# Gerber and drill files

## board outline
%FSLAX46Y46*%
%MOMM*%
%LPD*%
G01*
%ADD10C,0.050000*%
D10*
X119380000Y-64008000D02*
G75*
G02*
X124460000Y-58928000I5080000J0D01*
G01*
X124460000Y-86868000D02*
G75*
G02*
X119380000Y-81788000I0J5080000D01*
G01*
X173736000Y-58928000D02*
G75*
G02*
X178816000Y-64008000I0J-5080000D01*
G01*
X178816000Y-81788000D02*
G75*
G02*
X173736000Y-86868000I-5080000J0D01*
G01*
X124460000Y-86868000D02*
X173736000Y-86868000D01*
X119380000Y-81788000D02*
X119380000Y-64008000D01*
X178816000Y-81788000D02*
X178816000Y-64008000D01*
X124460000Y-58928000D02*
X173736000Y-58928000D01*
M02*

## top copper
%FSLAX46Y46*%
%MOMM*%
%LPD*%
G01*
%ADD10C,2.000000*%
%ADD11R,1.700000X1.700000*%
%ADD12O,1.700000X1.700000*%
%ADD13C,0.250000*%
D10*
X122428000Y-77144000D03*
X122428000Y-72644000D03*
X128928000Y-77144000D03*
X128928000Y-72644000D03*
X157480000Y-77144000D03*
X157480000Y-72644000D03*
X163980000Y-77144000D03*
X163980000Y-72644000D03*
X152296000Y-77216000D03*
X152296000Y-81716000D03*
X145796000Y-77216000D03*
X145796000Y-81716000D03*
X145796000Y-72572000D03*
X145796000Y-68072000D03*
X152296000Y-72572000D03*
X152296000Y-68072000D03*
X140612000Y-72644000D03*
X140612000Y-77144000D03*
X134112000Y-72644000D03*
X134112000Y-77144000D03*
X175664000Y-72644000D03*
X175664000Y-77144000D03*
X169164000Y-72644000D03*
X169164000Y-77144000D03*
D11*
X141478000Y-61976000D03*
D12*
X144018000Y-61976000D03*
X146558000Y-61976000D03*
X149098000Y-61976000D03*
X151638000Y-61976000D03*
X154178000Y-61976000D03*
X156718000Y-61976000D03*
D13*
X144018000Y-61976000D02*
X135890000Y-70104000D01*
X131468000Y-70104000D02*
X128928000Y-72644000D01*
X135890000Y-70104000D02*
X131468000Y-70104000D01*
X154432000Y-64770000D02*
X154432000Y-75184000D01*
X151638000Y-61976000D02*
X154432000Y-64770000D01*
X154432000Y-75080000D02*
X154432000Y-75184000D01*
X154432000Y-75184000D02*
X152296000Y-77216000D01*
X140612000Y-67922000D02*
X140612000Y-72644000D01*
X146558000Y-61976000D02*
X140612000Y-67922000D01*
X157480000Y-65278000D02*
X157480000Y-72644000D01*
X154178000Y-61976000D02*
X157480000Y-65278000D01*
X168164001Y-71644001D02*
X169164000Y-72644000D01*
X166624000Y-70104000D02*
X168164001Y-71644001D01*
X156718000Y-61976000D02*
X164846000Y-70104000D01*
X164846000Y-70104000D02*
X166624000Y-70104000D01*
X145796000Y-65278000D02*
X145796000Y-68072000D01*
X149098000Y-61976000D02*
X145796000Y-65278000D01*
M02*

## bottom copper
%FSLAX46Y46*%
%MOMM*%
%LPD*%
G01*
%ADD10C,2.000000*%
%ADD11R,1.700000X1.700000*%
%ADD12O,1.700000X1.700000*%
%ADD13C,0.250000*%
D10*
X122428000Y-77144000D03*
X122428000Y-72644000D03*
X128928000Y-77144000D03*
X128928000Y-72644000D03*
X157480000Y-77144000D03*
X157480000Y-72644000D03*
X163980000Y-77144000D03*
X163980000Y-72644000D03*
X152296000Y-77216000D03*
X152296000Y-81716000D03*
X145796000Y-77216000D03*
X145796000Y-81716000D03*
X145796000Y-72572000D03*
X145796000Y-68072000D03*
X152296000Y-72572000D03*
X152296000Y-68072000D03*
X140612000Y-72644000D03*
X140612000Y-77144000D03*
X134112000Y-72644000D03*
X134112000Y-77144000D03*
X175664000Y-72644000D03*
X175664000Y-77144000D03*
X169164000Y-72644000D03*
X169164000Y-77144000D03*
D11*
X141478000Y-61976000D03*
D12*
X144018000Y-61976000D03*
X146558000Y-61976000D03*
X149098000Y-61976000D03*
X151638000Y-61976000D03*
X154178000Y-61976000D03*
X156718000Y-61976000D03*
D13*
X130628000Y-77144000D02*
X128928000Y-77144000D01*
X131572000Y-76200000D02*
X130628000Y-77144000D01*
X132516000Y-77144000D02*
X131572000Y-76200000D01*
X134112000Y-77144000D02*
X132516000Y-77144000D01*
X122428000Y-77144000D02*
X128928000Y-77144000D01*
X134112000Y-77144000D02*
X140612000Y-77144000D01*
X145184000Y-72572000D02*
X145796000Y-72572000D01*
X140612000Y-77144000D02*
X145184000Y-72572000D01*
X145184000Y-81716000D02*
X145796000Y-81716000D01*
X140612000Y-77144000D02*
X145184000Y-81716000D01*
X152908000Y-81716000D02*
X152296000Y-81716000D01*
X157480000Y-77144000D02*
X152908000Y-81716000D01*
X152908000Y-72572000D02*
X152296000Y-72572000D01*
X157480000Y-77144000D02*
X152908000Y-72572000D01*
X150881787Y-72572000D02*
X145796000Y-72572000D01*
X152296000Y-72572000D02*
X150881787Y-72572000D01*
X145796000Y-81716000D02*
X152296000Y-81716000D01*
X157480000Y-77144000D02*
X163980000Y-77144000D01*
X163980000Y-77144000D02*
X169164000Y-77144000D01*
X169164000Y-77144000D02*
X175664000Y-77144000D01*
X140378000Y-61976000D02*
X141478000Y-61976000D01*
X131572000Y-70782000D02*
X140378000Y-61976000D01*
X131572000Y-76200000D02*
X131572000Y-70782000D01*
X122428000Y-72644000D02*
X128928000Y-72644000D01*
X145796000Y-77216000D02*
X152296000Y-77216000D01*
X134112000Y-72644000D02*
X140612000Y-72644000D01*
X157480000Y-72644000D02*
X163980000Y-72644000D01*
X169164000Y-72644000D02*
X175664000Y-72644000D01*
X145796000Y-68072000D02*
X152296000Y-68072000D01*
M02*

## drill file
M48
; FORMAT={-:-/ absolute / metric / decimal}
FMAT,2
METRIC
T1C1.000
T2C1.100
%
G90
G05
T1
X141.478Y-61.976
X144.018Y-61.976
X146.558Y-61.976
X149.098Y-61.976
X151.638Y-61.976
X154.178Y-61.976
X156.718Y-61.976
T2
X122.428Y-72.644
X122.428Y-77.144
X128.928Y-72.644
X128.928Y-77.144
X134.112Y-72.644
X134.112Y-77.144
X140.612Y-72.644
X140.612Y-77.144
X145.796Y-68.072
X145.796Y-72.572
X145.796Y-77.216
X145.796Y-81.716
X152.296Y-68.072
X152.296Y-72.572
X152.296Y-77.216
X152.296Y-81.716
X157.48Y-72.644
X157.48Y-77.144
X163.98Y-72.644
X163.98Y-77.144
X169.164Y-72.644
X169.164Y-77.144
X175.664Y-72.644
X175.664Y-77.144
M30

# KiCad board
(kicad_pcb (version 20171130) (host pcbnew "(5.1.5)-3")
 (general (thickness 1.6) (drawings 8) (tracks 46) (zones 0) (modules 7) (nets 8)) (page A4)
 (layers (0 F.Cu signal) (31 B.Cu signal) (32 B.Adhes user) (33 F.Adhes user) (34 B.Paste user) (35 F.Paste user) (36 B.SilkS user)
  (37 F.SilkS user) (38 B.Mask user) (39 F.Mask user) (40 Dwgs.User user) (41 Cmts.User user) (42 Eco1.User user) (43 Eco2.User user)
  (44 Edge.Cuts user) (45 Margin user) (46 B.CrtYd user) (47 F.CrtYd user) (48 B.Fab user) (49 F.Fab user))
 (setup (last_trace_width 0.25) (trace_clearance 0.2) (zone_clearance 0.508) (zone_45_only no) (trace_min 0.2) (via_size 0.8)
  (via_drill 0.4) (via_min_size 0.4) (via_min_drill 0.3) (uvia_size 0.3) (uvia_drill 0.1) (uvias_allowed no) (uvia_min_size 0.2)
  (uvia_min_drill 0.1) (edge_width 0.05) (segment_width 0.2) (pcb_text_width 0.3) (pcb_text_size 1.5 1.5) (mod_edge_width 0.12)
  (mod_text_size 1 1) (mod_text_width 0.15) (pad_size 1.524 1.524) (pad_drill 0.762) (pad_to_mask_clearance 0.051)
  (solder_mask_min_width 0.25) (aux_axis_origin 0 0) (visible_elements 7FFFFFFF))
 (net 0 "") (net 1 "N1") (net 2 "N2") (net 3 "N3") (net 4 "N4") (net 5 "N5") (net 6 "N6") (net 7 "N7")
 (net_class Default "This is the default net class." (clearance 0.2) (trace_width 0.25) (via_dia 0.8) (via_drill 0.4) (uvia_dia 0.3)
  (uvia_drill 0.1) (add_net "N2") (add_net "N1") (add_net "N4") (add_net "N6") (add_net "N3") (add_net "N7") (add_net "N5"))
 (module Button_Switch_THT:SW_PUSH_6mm (layer F.Cu) (at 122.428 72.644)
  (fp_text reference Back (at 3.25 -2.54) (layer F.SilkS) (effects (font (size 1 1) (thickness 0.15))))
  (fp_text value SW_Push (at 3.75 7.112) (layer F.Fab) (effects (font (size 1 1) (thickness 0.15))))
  (pad 2 thru_hole circle (at 0 4.5 90) (size 2 2) (drill 1.1) (layers *.Cu *.Mask) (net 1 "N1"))
  (pad 1 thru_hole circle (at 0 0 90) (size 2 2) (drill 1.1) (layers *.Cu *.Mask) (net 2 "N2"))
  (pad 2 thru_hole circle (at 6.5 4.5 90) (size 2 2) (drill 1.1) (layers *.Cu *.Mask) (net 1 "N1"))
  (pad 1 thru_hole circle (at 6.5 0 90) (size 2 2) (drill 1.1) (layers *.Cu *.Mask) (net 2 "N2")))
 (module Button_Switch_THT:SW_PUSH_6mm (layer F.Cu) (at 157.48 72.644)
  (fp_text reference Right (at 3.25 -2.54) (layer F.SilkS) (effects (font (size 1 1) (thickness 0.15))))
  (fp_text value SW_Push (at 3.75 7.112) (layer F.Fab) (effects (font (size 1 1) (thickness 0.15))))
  (pad 2 thru_hole circle (at 0 4.5 90) (size 2 2) (drill 1.1) (layers *.Cu *.Mask) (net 1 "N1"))
  (pad 1 thru_hole circle (at 0 0 90) (size 2 2) (drill 1.1) (layers *.Cu *.Mask) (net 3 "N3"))
  (pad 2 thru_hole circle (at 6.5 4.5 90) (size 2 2) (drill 1.1) (layers *.Cu *.Mask) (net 1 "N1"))
  (pad 1 thru_hole circle (at 6.5 0 90) (size 2 2) (drill 1.1) (layers *.Cu *.Mask) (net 3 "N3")))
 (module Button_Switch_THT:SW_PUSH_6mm (layer F.Cu) (at 145.796 77.216)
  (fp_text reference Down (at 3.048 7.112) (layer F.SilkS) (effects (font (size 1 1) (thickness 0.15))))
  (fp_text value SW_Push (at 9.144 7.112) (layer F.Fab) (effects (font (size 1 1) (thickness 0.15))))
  (pad 1 thru_hole circle (at 6.5 0 90) (size 2 2) (drill 1.1) (layers *.Cu *.Mask) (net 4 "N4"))
  (pad 2 thru_hole circle (at 6.5 4.5 90) (size 2 2) (drill 1.1) (layers *.Cu *.Mask) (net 1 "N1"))
  (pad 1 thru_hole circle (at 0 0 90) (size 2 2) (drill 1.1) (layers *.Cu *.Mask) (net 4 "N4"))
  (pad 2 thru_hole circle (at 0 4.5 90) (size 2 2) (drill 1.1) (layers *.Cu *.Mask) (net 1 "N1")))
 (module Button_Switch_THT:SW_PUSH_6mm (layer F.Cu) (at 145.796 68.072)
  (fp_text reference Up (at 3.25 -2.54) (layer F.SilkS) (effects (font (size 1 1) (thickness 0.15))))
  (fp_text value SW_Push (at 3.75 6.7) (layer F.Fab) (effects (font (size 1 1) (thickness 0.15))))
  (pad 2 thru_hole circle (at 0 4.5 90) (size 2 2) (drill 1.1) (layers *.Cu *.Mask) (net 1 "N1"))
  (pad 1 thru_hole circle (at 0 0 90) (size 2 2) (drill 1.1) (layers *.Cu *.Mask) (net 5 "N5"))
  (pad 2 thru_hole circle (at 6.5 4.5 90) (size 2 2) (drill 1.1) (layers *.Cu *.Mask) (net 1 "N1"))
  (pad 1 thru_hole circle (at 6.5 0 90) (size 2 2) (drill 1.1) (layers *.Cu *.Mask) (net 5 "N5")))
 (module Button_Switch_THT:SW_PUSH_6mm (layer F.Cu) (at 134.112 72.644)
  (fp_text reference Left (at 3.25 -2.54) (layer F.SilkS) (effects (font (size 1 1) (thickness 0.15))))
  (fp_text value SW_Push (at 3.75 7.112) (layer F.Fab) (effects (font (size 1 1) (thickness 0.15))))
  (pad 1 thru_hole circle (at 6.5 0 90) (size 2 2) (drill 1.1) (layers *.Cu *.Mask) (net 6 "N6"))
  (pad 2 thru_hole circle (at 6.5 4.5 90) (size 2 2) (drill 1.1) (layers *.Cu *.Mask) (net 1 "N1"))
  (pad 1 thru_hole circle (at 0 0 90) (size 2 2) (drill 1.1) (layers *.Cu *.Mask) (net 6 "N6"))
  (pad 2 thru_hole circle (at 0 4.5 90) (size 2 2) (drill 1.1) (layers *.Cu *.Mask) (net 1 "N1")))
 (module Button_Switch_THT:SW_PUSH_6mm (layer F.Cu) (at 169.164 72.644)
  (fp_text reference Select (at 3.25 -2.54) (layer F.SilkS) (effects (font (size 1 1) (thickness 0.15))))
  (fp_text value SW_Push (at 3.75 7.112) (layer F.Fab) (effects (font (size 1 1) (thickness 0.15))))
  (pad 1 thru_hole circle (at 6.5 0 90) (size 2 2) (drill 1.1) (layers *.Cu *.Mask) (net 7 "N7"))
  (pad 2 thru_hole circle (at 6.5 4.5 90) (size 2 2) (drill 1.1) (layers *.Cu *.Mask) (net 1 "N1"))
  (pad 1 thru_hole circle (at 0 0 90) (size 2 2) (drill 1.1) (layers *.Cu *.Mask) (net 7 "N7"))
  (pad 2 thru_hole circle (at 0 4.5 90) (size 2 2) (drill 1.1) (layers *.Cu *.Mask) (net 1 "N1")))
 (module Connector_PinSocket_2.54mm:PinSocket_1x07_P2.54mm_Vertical (layer F.Cu) (at 141.478 61.976 90)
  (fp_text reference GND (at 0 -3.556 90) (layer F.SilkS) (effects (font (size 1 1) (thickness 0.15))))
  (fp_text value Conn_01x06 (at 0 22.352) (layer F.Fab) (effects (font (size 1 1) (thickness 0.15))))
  (pad 1 thru_hole rect (at 0 0 90) (size 1.7 1.7) (drill 1) (layers *.Cu *.Mask) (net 1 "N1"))
  (pad 2 thru_hole oval (at 0 2.54 90) (size 1.7 1.7) (drill 1) (layers *.Cu *.Mask) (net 2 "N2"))
  (pad 3 thru_hole oval (at 0 5.08 90) (size 1.7 1.7) (drill 1) (layers *.Cu *.Mask) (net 6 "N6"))
  (pad 4 thru_hole oval (at 0 7.62 90) (size 1.7 1.7) (drill 1) (layers *.Cu *.Mask) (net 5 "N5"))
  (pad 5 thru_hole oval (at 0 10.16 90) (size 1.7 1.7) (drill 1) (layers *.Cu *.Mask) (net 4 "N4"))
  (pad 6 thru_hole oval (at 0 12.7 90) (size 1.7 1.7) (drill 1) (layers *.Cu *.Mask) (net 3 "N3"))
  (pad 7 thru_hole oval (at 0 15.24 90) (size 1.7 1.7) (drill 1) (layers *.Cu *.Mask) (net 7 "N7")))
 (gr_arc (start 124.46 64.008) (end 124.46 58.928) (angle -90) (layer Edge.Cuts) (width 0.05))
 (gr_arc (start 124.46 81.788) (end 119.38 81.788) (angle -90) (layer Edge.Cuts) (width 0.05))
 (gr_arc (start 173.736 64.008) (end 178.816 64.008) (angle -90) (layer Edge.Cuts) (width 0.05))
 (gr_arc (start 173.736 81.788) (end 173.736 86.868) (angle -90) (layer Edge.Cuts) (width 0.05))
 (gr_line (start 124.46 86.868) (end 173.736 86.868) (layer Edge.Cuts) (width 0.05))
 (gr_line (start 119.38 81.788) (end 119.38 64.008) (layer Edge.Cuts) (width 0.05))
 (gr_line (start 178.816 81.788) (end 178.816 64.008) (layer Edge.Cuts) (width 0.05))
 (gr_line (start 124.46 58.928) (end 173.736 58.928) (layer Edge.Cuts) (width 0.05))
 (segment (start 130.628 77.144) (end 128.928 77.144) (width 0.25) (layer B.Cu) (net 1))
 (segment (start 131.572 76.2) (end 130.628 77.144) (width 0.25) (layer B.Cu) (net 1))
 (segment (start 132.516 77.144) (end 131.572 76.2) (width 0.25) (layer B.Cu) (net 1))
 (segment (start 134.112 77.144) (end 132.516 77.144) (width 0.25) (layer B.Cu) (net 1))
 (segment (start 122.428 77.144) (end 128.928 77.144) (width 0.25) (layer B.Cu) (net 1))
 (segment (start 134.112 77.144) (end 140.612 77.144) (width 0.25) (layer B.Cu) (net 1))
 (segment (start 145.184 72.572) (end 145.796 72.572) (width 0.25) (layer B.Cu) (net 1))
 (segment (start 140.612 77.144) (end 145.184 72.572) (width 0.25) (layer B.Cu) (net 1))
 (segment (start 145.184 81.716) (end 145.796 81.716) (width 0.25) (layer B.Cu) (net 1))
 (segment (start 140.612 77.144) (end 145.184 81.716) (width 0.25) (layer B.Cu) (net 1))
 (segment (start 152.908 81.716) (end 152.296 81.716) (width 0.25) (layer B.Cu) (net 1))
 (segment (start 157.48 77.144) (end 152.908 81.716) (width 0.25) (layer B.Cu) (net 1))
 (segment (start 152.908 72.572) (end 152.296 72.572) (width 0.25) (layer B.Cu) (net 1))
 (segment (start 157.48 77.144) (end 152.908 72.572) (width 0.25) (layer B.Cu) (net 1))
 (segment (start 150.881787 72.572) (end 145.796 72.572) (width 0.25) (layer B.Cu) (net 1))
 (segment (start 152.296 72.572) (end 150.881787 72.572) (width 0.25) (layer B.Cu) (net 1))
 (segment (start 145.796 81.716) (end 152.296 81.716) (width 0.25) (layer B.Cu) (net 1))
 (segment (start 157.48 77.144) (end 163.98 77.144) (width 0.25) (layer B.Cu) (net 1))
 (segment (start 163.98 77.144) (end 169.164 77.144) (width 0.25) (layer B.Cu) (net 1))
 (segment (start 169.164 77.144) (end 175.664 77.144) (width 0.25) (layer B.Cu) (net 1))
 (segment (start 140.378 61.976) (end 141.478 61.976) (width 0.25) (layer B.Cu) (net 1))
 (segment (start 131.572 70.782) (end 140.378 61.976) (width 0.25) (layer B.Cu) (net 1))
 (segment (start 131.572 76.2) (end 131.572 70.782) (width 0.25) (layer B.Cu) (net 1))
 (segment (start 122.428 72.644) (end 128.928 72.644) (width 0.25) (layer B.Cu) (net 2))
 (segment (start 144.018 61.976) (end 135.89 70.104) (width 0.25) (layer F.Cu) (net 2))
 (segment (start 131.468 70.104) (end 128.928 72.644) (width 0.25) (layer F.Cu) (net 2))
 (segment (start 135.89 70.104) (end 131.468 70.104) (width 0.25) (layer F.Cu) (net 2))
 (segment (start 145.796 77.216) (end 152.296 77.216) (width 0.25) (layer B.Cu) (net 4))
 (segment (start 154.432 64.77) (end 154.432 75.184) (width 0.25) (layer F.Cu) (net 4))
 (segment (start 151.638 61.976) (end 154.432 64.77) (width 0.25) (layer F.Cu) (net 4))
 (segment (start 154.432 75.08) (end 154.432 75.184) (width 0.25) (layer F.Cu) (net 4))
 (segment (start 154.432 75.184) (end 152.296 77.216) (width 0.25) (layer F.Cu) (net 4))
 (segment (start 134.112 72.644) (end 140.612 72.644) (width 0.25) (layer B.Cu) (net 6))
 (segment (start 140.612 67.922) (end 140.612 72.644) (width 0.25) (layer F.Cu) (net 6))
 (segment (start 146.558 61.976) (end 140.612 67.922) (width 0.25) (layer F.Cu) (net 6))
 (segment (start 157.48 72.644) (end 163.98 72.644) (width 0.25) (layer B.Cu) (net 3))
 (segment (start 157.48 65.278) (end 157.48 72.644) (width 0.25) (layer F.Cu) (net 3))
 (segment (start 154.178 61.976) (end 157.48 65.278) (width 0.25) (layer F.Cu) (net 3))
 (segment (start 169.164 72.644) (end 175.664 72.644) (width 0.25) (layer B.Cu) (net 7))
 (segment (start 168.164001 71.644001) (end 169.164 72.644) (width 0.25) (layer F.Cu) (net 7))
 (segment (start 166.624 70.104) (end 168.164001 71.644001) (width 0.25) (layer F.Cu) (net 7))
 (segment (start 156.718 61.976) (end 164.846 70.104) (width 0.25) (layer F.Cu) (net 7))
 (segment (start 164.846 70.104) (end 166.624 70.104) (width 0.25) (layer F.Cu) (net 7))
 (segment (start 145.796 68.072) (end 152.296 68.072) (width 0.25) (layer B.Cu) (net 5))
 (segment (start 145.796 65.278) (end 145.796 68.072) (width 0.25) (layer F.Cu) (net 5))
 (segment (start 149.098 61.976) (end 145.796 65.278) (width 0.25) (layer F.Cu) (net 5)))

